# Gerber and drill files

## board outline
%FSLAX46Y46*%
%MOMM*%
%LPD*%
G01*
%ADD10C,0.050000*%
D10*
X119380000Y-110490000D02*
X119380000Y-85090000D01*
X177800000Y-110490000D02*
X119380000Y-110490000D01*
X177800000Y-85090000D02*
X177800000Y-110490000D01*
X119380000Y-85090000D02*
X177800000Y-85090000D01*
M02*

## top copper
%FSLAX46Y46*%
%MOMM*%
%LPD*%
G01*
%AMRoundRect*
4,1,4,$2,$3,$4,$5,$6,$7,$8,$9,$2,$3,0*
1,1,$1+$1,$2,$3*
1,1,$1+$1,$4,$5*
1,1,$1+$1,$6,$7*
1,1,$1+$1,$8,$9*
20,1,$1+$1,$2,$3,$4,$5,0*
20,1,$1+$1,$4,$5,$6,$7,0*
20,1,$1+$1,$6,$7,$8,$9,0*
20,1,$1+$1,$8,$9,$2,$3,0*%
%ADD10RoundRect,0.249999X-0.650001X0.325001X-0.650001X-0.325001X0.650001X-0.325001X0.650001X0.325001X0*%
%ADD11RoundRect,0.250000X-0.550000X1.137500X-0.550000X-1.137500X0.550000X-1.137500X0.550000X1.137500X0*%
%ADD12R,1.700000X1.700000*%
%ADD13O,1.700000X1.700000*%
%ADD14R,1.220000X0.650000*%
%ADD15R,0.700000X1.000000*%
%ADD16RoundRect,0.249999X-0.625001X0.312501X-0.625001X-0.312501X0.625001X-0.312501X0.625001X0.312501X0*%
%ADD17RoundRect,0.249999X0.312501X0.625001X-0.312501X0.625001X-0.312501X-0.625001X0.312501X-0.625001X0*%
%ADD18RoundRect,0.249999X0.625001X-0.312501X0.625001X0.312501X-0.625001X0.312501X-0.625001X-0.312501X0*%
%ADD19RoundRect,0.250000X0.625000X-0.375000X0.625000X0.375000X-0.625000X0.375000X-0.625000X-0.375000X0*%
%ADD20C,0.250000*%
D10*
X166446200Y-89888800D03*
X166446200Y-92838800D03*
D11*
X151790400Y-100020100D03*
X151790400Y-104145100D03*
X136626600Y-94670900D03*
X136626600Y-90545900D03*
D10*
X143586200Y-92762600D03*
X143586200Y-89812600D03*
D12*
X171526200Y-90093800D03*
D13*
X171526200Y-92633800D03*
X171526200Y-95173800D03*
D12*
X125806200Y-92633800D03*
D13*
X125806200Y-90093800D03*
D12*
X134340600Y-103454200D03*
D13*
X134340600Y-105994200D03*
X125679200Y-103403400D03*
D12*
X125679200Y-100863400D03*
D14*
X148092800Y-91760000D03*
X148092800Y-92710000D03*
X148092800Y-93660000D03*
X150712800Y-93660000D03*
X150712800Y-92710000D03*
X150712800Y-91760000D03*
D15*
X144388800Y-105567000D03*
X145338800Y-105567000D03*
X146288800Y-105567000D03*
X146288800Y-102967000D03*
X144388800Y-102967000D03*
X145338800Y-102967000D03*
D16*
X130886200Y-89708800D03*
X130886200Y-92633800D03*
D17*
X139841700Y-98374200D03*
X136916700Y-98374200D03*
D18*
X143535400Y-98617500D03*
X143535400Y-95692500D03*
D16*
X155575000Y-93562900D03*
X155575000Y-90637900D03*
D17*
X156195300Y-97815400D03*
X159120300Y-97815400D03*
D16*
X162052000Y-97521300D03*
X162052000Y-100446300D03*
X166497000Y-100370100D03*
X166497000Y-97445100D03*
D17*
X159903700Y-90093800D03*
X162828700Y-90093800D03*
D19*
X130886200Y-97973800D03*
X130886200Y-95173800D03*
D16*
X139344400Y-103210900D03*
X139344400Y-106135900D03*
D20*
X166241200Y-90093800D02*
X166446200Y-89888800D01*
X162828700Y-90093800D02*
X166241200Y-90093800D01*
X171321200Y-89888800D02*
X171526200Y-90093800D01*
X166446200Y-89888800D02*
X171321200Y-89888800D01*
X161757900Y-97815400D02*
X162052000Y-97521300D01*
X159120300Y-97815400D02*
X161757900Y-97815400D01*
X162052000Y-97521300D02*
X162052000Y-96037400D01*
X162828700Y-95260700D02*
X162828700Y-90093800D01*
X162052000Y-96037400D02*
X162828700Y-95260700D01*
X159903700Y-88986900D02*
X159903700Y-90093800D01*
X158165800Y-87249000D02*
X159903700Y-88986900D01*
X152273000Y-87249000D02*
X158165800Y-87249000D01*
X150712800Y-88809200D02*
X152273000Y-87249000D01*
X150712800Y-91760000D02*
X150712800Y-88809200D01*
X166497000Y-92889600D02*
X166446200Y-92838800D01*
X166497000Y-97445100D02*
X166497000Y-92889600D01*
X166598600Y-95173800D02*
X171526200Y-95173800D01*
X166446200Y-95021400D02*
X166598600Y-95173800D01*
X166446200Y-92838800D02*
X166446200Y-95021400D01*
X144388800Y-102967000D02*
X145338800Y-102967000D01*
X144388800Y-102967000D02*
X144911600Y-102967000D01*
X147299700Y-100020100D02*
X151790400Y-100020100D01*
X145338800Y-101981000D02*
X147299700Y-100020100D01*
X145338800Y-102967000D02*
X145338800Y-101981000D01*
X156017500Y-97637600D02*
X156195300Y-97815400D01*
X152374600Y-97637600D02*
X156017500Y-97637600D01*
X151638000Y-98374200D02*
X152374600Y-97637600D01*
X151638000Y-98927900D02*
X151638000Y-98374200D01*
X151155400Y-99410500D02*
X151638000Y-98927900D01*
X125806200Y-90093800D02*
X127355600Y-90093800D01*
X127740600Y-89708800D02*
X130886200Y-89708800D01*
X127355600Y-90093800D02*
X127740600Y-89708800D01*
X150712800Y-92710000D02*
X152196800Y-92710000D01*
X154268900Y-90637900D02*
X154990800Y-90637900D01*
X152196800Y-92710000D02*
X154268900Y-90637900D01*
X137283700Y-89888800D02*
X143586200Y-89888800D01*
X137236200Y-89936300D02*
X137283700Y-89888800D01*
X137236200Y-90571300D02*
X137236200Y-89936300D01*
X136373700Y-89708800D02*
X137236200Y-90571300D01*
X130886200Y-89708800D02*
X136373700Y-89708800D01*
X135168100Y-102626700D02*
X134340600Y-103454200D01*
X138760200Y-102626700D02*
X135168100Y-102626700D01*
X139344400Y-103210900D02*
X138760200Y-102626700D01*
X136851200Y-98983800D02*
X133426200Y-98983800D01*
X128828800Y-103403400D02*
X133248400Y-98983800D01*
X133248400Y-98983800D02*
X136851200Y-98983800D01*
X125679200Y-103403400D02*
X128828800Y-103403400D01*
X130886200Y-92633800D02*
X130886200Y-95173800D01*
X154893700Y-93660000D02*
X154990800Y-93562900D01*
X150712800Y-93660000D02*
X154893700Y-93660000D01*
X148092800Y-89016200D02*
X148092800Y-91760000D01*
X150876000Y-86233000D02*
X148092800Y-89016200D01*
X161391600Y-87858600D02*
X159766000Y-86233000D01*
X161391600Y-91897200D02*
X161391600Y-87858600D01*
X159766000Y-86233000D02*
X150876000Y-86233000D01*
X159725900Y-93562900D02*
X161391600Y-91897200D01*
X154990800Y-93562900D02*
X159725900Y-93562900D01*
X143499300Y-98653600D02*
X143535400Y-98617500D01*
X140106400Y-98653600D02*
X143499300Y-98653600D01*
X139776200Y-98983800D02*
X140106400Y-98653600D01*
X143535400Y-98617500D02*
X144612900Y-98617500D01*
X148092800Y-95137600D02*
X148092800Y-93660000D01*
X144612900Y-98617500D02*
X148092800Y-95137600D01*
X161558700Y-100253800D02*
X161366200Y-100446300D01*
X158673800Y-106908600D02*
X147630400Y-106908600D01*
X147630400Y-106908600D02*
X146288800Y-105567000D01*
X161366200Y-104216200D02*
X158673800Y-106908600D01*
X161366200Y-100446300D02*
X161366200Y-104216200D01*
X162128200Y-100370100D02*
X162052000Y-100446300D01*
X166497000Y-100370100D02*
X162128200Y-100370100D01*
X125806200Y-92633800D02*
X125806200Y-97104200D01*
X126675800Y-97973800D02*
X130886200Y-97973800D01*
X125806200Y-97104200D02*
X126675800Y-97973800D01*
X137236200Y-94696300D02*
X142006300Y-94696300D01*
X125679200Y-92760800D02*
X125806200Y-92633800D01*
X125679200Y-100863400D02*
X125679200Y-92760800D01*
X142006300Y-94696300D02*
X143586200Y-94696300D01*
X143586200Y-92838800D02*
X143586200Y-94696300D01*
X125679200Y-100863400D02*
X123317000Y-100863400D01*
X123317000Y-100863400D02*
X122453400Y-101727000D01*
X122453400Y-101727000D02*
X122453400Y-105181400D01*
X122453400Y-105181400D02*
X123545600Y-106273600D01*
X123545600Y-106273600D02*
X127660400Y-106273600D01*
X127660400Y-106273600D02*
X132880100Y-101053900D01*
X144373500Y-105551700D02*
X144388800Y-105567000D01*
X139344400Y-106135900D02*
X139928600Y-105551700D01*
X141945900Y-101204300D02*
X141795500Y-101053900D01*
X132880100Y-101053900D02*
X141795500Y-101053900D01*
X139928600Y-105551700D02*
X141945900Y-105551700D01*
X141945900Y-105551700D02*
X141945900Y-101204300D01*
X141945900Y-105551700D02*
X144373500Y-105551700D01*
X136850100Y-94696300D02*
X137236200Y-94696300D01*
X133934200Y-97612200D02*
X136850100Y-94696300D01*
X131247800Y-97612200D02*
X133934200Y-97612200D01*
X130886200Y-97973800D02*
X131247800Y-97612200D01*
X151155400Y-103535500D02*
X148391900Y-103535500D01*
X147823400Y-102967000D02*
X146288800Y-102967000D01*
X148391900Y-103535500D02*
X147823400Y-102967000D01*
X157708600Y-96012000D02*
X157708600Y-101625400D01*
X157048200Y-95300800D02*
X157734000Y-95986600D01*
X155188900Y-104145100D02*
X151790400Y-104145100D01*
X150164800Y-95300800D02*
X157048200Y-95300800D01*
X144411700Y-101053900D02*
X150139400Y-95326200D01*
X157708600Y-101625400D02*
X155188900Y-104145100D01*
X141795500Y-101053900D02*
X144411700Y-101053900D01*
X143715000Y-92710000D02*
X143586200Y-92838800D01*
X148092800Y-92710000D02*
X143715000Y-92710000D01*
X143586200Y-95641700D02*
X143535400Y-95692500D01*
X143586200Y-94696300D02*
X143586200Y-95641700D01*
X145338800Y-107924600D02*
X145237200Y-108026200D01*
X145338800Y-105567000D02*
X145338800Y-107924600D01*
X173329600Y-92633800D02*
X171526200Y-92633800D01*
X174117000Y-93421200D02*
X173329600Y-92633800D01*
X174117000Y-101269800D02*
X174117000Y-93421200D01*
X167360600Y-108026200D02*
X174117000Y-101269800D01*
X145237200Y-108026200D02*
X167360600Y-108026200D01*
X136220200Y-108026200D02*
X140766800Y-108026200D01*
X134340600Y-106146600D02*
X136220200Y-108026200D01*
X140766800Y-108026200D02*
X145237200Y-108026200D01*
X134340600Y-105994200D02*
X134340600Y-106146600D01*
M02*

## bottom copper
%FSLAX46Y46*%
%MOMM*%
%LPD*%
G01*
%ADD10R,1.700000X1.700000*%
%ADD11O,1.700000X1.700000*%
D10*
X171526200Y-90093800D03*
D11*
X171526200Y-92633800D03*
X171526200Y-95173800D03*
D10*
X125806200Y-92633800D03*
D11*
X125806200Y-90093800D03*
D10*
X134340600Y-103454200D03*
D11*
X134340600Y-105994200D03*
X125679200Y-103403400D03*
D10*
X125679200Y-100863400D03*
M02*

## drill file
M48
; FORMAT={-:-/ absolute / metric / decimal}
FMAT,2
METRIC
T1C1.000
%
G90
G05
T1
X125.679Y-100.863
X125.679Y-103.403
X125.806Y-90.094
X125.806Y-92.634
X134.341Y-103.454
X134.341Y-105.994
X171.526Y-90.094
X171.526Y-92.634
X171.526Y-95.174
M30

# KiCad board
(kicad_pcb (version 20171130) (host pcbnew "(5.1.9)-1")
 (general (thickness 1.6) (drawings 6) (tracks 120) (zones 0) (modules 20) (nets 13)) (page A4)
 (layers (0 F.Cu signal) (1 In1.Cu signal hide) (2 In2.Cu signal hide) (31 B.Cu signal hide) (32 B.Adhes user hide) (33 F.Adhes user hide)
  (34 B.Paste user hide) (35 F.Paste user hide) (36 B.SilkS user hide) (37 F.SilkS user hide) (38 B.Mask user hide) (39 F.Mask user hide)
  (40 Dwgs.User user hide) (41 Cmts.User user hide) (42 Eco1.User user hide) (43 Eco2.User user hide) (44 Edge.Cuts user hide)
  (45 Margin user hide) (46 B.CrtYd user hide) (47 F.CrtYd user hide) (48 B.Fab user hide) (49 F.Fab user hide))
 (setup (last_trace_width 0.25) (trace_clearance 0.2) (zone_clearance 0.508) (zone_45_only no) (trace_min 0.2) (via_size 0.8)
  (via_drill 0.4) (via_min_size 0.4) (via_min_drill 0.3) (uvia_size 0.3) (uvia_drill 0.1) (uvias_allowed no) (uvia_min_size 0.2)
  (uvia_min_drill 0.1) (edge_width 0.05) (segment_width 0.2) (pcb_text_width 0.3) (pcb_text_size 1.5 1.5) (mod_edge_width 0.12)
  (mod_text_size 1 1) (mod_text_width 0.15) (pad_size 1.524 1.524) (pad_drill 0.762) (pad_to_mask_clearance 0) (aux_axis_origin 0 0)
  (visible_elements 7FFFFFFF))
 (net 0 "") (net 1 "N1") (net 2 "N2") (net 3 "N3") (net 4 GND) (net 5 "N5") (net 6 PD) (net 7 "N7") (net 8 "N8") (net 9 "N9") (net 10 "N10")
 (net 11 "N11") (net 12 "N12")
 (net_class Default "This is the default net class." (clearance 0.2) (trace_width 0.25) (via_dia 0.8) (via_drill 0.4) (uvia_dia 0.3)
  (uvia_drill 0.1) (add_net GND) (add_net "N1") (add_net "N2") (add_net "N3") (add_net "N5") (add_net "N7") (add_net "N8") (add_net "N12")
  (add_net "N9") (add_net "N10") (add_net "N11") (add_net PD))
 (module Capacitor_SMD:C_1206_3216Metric (layer F.Cu) (at 166.4462 91.3638 270)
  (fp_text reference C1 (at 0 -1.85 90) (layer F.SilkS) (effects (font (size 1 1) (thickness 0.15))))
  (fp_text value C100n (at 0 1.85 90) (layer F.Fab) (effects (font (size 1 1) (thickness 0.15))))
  (pad 1 smd roundrect (at -1.475 0 270) (size 1.15 1.8) (layers F.Cu F.Paste F.Mask) (roundrect_rratio 0.2173904347826087) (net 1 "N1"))
  (pad 2 smd roundrect (at 1.475 0 270) (size 1.15 1.8) (layers F.Cu F.Paste F.Mask) (roundrect_rratio 0.2173904347826087) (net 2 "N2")))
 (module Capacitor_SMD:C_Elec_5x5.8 (layer F.Cu) (at 151.7904 102.0826 270)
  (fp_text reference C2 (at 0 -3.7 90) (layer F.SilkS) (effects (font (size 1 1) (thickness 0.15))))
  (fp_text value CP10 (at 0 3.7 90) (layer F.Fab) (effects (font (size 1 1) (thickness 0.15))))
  (pad 1 smd roundrect (at -2.0625 0 270) (size 2.775 1.6) (layers F.Cu F.Paste F.Mask) (roundrect_rratio 0.15625) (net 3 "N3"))
  (pad 2 smd roundrect (at 2.0625 0 270) (size 2.775 1.6) (layers F.Cu F.Paste F.Mask) (roundrect_rratio 0.15625) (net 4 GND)))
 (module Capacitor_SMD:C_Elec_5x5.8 (layer F.Cu) (at 136.6266 92.6084 270)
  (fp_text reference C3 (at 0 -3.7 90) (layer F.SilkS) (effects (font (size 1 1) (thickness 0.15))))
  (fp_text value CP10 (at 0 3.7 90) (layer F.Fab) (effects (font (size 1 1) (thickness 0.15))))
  (pad 2 smd roundrect (at 2.0625 0 270) (size 2.775 1.6) (layers F.Cu F.Paste F.Mask) (roundrect_rratio 0.15625) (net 4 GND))
  (pad 1 smd roundrect (at -2.0625 0 270) (size 2.775 1.6) (layers F.Cu F.Paste F.Mask) (roundrect_rratio 0.15625) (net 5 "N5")))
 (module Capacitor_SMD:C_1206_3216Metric (layer F.Cu) (at 143.5862 91.2876 270)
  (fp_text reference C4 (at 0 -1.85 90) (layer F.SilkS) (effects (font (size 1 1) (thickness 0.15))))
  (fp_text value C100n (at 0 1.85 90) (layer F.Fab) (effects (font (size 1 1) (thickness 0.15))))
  (pad 2 smd roundrect (at 1.475 0 270) (size 1.15 1.8) (layers F.Cu F.Paste F.Mask) (roundrect_rratio 0.2173904347826087) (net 4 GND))
  (pad 1 smd roundrect (at -1.475 0 270) (size 1.15 1.8) (layers F.Cu F.Paste F.Mask) (roundrect_rratio 0.2173904347826087) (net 5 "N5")))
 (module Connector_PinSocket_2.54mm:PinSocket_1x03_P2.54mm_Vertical (layer F.Cu) (at 171.5262 90.0938)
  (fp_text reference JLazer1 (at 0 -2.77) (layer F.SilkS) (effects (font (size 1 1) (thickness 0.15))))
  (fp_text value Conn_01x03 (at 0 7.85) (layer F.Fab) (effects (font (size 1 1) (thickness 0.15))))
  (pad 1 thru_hole rect (at 0 0) (size 1.7 1.7) (drill 1) (layers *.Cu *.Mask) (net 1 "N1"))
  (pad 2 thru_hole oval (at 0 2.54) (size 1.7 1.7) (drill 1) (layers *.Cu *.Mask) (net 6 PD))
  (pad 3 thru_hole oval (at 0 5.08) (size 1.7 1.7) (drill 1) (layers *.Cu *.Mask) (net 2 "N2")))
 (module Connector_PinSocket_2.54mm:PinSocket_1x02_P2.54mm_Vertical (layer F.Cu) (at 125.8062 92.6338 180)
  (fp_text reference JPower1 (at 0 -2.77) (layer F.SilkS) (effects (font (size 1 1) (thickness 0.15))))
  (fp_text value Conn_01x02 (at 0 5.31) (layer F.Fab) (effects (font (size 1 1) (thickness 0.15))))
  (pad 1 thru_hole rect (at 0 0 180) (size 1.7 1.7) (drill 1) (layers *.Cu *.Mask) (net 4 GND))
  (pad 2 thru_hole oval (at 0 2.54 180) (size 1.7 1.7) (drill 1) (layers *.Cu *.Mask) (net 5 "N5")))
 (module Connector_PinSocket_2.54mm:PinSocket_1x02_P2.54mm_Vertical (layer F.Cu) (at 134.3406 103.4542)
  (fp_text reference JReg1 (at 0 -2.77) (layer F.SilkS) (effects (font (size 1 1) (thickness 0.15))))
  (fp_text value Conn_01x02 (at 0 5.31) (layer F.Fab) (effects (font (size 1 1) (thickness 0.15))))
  (pad 1 thru_hole rect (at 0 0) (size 1.7 1.7) (drill 1) (layers *.Cu *.Mask) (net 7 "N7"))
  (pad 2 thru_hole oval (at 0 2.54) (size 1.7 1.7) (drill 1) (layers *.Cu *.Mask) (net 6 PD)))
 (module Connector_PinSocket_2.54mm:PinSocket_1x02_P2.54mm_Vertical (layer F.Cu) (at 125.6792 100.8634)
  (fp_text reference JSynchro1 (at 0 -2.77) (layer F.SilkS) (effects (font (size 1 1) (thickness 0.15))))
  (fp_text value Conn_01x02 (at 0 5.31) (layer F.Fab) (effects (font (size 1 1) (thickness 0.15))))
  (pad 2 thru_hole oval (at 0 2.54) (size 1.7 1.7) (drill 1) (layers *.Cu *.Mask) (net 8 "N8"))
  (pad 1 thru_hole rect (at 0 0) (size 1.7 1.7) (drill 1) (layers *.Cu *.Mask) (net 4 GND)))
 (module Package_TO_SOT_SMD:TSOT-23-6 (layer F.Cu) (at 149.4028 92.71)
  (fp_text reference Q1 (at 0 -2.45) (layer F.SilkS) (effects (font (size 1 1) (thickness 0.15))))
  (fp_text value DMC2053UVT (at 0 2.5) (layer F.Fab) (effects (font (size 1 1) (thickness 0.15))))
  (pad 1 smd rect (at -1.31 -0.95) (size 1.22 0.65) (layers F.Cu F.Paste F.Mask) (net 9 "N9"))
  (pad 2 smd rect (at -1.31 0) (size 1.22 0.65) (layers F.Cu F.Paste F.Mask) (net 4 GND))
  (pad 3 smd rect (at -1.31 0.95) (size 1.22 0.65) (layers F.Cu F.Paste F.Mask) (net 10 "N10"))
  (pad 4 smd rect (at 1.31 0.95) (size 1.22 0.65) (layers F.Cu F.Paste F.Mask) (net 9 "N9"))
  (pad 5 smd rect (at 1.31 0) (size 1.22 0.65) (layers F.Cu F.Paste F.Mask) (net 5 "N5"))
  (pad 6 smd rect (at 1.31 -0.95) (size 1.22 0.65) (layers F.Cu F.Paste F.Mask) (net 1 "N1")))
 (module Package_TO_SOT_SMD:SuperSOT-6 (layer F.Cu) (at 145.3388 104.267 90)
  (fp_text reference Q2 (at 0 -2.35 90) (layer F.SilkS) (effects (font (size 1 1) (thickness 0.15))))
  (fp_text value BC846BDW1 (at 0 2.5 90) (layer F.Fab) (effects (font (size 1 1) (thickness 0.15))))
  (pad 1 smd rect (at -1.3 -0.95 90) (size 1 0.7) (layers F.Cu F.Paste F.Mask) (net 4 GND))
  (pad 2 smd rect (at -1.3 0 90) (size 1 0.7) (layers F.Cu F.Paste F.Mask) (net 6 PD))
  (pad 3 smd rect (at -1.3 0.95 90) (size 1 0.7) (layers F.Cu F.Paste F.Mask) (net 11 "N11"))
  (pad 4 smd rect (at 1.3 0.95 90) (size 1 0.7) (layers F.Cu F.Paste F.Mask) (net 4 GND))
  (pad 6 smd rect (at 1.3 -0.95 90) (size 1 0.7) (layers F.Cu F.Paste F.Mask) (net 3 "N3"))
  (pad 5 smd rect (at 1.3 0 90) (size 1 0.7) (layers F.Cu F.Paste F.Mask) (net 3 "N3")))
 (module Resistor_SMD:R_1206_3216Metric (layer F.Cu) (at 130.8862 91.1713 270)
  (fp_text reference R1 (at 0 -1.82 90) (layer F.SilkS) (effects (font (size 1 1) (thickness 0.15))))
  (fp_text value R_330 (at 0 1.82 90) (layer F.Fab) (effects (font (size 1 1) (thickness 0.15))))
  (pad 1 smd roundrect (at -1.4625 0 270) (size 1.125 1.75) (layers F.Cu F.Paste F.Mask) (roundrect_rratio 0.2222213333333333) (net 5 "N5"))
  (pad 2 smd roundrect (at 1.4625 0 270) (size 1.125 1.75) (layers F.Cu F.Paste F.Mask) (roundrect_rratio 0.2222213333333333) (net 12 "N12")))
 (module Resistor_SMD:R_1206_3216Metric (layer F.Cu) (at 138.3792 98.3742 180)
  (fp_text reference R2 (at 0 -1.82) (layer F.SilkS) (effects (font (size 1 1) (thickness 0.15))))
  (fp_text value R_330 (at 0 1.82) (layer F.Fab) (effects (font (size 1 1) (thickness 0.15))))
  (pad 1 smd roundrect (at -1.4625 0 180) (size 1.125 1.75) (layers F.Cu F.Paste F.Mask) (roundrect_rratio 0.2222213333333333)
   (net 10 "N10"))
  (pad 2 smd roundrect (at 1.4625 0 180) (size 1.125 1.75) (layers F.Cu F.Paste F.Mask) (roundrect_rratio 0.2222213333333333) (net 8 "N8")))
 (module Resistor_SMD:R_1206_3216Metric (layer F.Cu) (at 143.5354 97.155 90)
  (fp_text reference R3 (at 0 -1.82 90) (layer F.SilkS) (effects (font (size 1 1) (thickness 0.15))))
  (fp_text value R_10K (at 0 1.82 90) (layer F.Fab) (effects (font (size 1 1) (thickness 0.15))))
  (pad 1 smd roundrect (at -1.4625 0 90) (size 1.125 1.75) (layers F.Cu F.Paste F.Mask) (roundrect_rratio 0.2222213333333333) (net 10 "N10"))
  (pad 2 smd roundrect (at 1.4625 0 90) (size 1.125 1.75) (layers F.Cu F.Paste F.Mask) (roundrect_rratio 0.2222213333333333) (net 4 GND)))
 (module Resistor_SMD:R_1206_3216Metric (layer F.Cu) (at 155.575 92.1004 270)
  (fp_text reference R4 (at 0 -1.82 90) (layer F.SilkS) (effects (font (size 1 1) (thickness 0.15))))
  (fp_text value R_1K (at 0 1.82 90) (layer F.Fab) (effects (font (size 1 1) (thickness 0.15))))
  (pad 2 smd roundrect (at 1.4625 0 270) (size 1.125 1.75) (layers F.Cu F.Paste F.Mask) (roundrect_rratio 0.2222213333333333) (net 9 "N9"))
  (pad 1 smd roundrect (at -1.4625 0 270) (size 1.125 1.75) (layers F.Cu F.Paste F.Mask) (roundrect_rratio 0.2222213333333333) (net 5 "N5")))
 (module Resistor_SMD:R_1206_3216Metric (layer F.Cu) (at 157.6578 97.8154 180)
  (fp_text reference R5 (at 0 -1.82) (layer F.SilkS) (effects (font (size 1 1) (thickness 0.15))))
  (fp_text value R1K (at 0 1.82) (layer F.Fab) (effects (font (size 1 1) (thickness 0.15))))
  (pad 2 smd roundrect (at 1.4625 0 180) (size 1.125 1.75) (layers F.Cu F.Paste F.Mask) (roundrect_rratio 0.2222213333333333) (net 3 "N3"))
  (pad 1 smd roundrect (at -1.4625 0 180) (size 1.125 1.75) (layers F.Cu F.Paste F.Mask) (roundrect_rratio 0.2222213333333333) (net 1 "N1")))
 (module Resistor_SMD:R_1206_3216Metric (layer F.Cu) (at 162.052 98.9838 270)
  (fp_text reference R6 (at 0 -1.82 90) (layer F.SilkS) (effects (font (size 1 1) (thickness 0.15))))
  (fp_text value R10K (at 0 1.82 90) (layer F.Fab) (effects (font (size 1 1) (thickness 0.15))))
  (pad 1 smd roundrect (at -1.4625 0 270) (size 1.125 1.75) (layers F.Cu F.Paste F.Mask) (roundrect_rratio 0.2222213333333333) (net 1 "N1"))
  (pad 2 smd roundrect (at 1.4625 0 270) (size 1.125 1.75) (layers F.Cu F.Paste F.Mask) (roundrect_rratio 0.2222213333333333) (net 11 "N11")))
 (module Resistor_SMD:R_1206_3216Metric (layer F.Cu) (at 166.497 98.9076 270)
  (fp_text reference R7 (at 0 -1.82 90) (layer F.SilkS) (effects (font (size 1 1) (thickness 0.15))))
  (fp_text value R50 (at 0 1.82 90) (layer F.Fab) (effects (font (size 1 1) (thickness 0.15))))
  (pad 2 smd roundrect (at 1.4625 0 270) (size 1.125 1.75) (layers F.Cu F.Paste F.Mask) (roundrect_rratio 0.2222213333333333) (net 11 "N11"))
  (pad 1 smd roundrect (at -1.4625 0 270) (size 1.125 1.75) (layers F.Cu F.Paste F.Mask) (roundrect_rratio 0.2222213333333333) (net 2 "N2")))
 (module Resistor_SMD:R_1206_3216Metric (layer F.Cu) (at 161.3662 90.0938 180)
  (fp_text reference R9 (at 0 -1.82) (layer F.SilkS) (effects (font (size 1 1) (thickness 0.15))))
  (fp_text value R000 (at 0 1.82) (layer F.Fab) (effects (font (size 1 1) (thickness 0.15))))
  (pad 2 smd roundrect (at 1.4625 0 180) (size 1.125 1.75) (layers F.Cu F.Paste F.Mask) (roundrect_rratio 0.2222213333333333) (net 1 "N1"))
  (pad 1 smd roundrect (at -1.4625 0 180) (size 1.125 1.75) (layers F.Cu F.Paste F.Mask) (roundrect_rratio 0.2222213333333333) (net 1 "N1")))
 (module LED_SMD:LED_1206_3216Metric (layer F.Cu) (at 130.8862 96.5738 90)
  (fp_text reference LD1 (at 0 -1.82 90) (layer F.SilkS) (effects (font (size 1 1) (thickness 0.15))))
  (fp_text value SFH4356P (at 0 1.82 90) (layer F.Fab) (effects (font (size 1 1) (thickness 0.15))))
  (pad 1 smd roundrect (at -1.4 0 90) (size 1.25 1.75) (layers F.Cu F.Paste F.Mask) (roundrect_rratio 0.2) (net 4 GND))
  (pad 2 smd roundrect (at 1.4 0 90) (size 1.25 1.75) (layers F.Cu F.Paste F.Mask) (roundrect_rratio 0.2) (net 12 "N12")))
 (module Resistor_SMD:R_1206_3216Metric (layer F.Cu) (at 139.3444 104.6734 270)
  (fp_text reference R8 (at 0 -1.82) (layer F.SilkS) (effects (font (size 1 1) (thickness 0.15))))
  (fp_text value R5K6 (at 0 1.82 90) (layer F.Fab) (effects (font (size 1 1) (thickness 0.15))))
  (pad 1 smd roundrect (at -1.4625 0 270) (size 1.125 1.75) (layers F.Cu F.Paste F.Mask) (roundrect_rratio 0.2222213333333333) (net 7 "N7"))
  (pad 2 smd roundrect (at 1.4625 0 270) (size 1.125 1.75) (layers F.Cu F.Paste F.Mask) (roundrect_rratio 0.2222213333333333) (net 4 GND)))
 (gr_line (start 119.38 110.49) (end 119.38 85.09) (layer Edge.Cuts) (width 0.05))
 (gr_line (start 177.8 110.49) (end 119.38 110.49) (layer Edge.Cuts) (width 0.05))
 (gr_line (start 177.8 85.09) (end 177.8 110.49) (layer Edge.Cuts) (width 0.05))
 (gr_line (start 119.38 85.09) (end 177.8 85.09) (layer Edge.Cuts) (width 0.05))
 (segment (start 166.2412 90.0938) (end 166.4462 89.8888) (width 0.25) (layer F.Cu) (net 1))
 (segment (start 162.8287 90.0938) (end 166.2412 90.0938) (width 0.25) (layer F.Cu) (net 1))
 (segment (start 171.3212 89.8888) (end 171.5262 90.0938) (width 0.25) (layer F.Cu) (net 1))
 (segment (start 166.4462 89.8888) (end 171.3212 89.8888) (width 0.25) (layer F.Cu) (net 1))
 (segment (start 161.7579 97.8154) (end 162.052 97.5213) (width 0.25) (layer F.Cu) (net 1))
 (segment (start 159.1203 97.8154) (end 161.7579 97.8154) (width 0.25) (layer F.Cu) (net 1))
 (segment (start 162.052 97.5213) (end 162.052 96.0374) (width 0.25) (layer F.Cu) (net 1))
 (segment (start 162.8287 95.2607) (end 162.8287 90.0938) (width 0.25) (layer F.Cu) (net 1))
 (segment (start 162.052 96.0374) (end 162.8287 95.2607) (width 0.25) (layer F.Cu) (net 1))
 (segment (start 159.9037 88.9869) (end 159.9037 90.0938) (width 0.25) (layer F.Cu) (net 1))
 (segment (start 158.1658 87.249) (end 159.9037 88.9869) (width 0.25) (layer F.Cu) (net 1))
 (segment (start 152.273 87.249) (end 158.1658 87.249) (width 0.25) (layer F.Cu) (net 1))
 (segment (start 150.7128 88.8092) (end 152.273 87.249) (width 0.25) (layer F.Cu) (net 1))
 (segment (start 150.7128 91.76) (end 150.7128 88.8092) (width 0.25) (layer F.Cu) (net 1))
 (segment (start 166.497 92.8896) (end 166.4462 92.8388) (width 0.25) (layer F.Cu) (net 2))
 (segment (start 166.497 97.4451) (end 166.497 92.8896) (width 0.25) (layer F.Cu) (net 2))
 (segment (start 166.5986 95.1738) (end 171.5262 95.1738) (width 0.25) (layer F.Cu) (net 2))
 (segment (start 166.4462 95.0214) (end 166.5986 95.1738) (width 0.25) (layer F.Cu) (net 2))
 (segment (start 166.4462 92.8388) (end 166.4462 95.0214) (width 0.25) (layer F.Cu) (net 2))
 (segment (start 144.3888 102.967) (end 145.3388 102.967) (width 0.25) (layer F.Cu) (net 3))
 (segment (start 144.3888 102.967) (end 144.9116 102.967) (width 0.25) (layer F.Cu) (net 3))
 (segment (start 147.2997 100.0201) (end 151.7904 100.0201) (width 0.25) (layer F.Cu) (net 3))
 (segment (start 145.3388 101.981) (end 147.2997 100.0201) (width 0.25) (layer F.Cu) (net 3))
 (segment (start 145.3388 102.967) (end 145.3388 101.981) (width 0.25) (layer F.Cu) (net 3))
 (segment (start 156.0175 97.6376) (end 156.1953 97.8154) (width 0.25) (layer F.Cu) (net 3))
 (segment (start 152.3746 97.6376) (end 156.0175 97.6376) (width 0.25) (layer F.Cu) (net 3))
 (segment (start 151.638 98.3742) (end 152.3746 97.6376) (width 0.25) (layer F.Cu) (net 3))
 (segment (start 151.638 98.9279) (end 151.638 98.3742) (width 0.25) (layer F.Cu) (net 3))
 (segment (start 151.1554 99.4105) (end 151.638 98.9279) (width 0.25) (layer F.Cu) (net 3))
 (segment (start 125.8062 90.0938) (end 127.3556 90.0938) (width 0.25) (layer F.Cu) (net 5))
 (segment (start 127.7406 89.7088) (end 130.8862 89.7088) (width 0.25) (layer F.Cu) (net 5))
 (segment (start 127.3556 90.0938) (end 127.7406 89.7088) (width 0.25) (layer F.Cu) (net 5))
 (segment (start 150.7128 92.71) (end 152.1968 92.71) (width 0.25) (layer F.Cu) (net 5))
 (segment (start 154.2689 90.6379) (end 154.9908 90.6379) (width 0.25) (layer F.Cu) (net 5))
 (segment (start 152.1968 92.71) (end 154.2689 90.6379) (width 0.25) (layer F.Cu) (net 5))
 (segment (start 137.2837 89.8888) (end 143.5862 89.8888) (width 0.25) (layer F.Cu) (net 5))
 (segment (start 137.2362 89.9363) (end 137.2837 89.8888) (width 0.25) (layer F.Cu) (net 5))
 (segment (start 137.2362 90.5713) (end 137.2362 89.9363) (width 0.25) (layer F.Cu) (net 5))
 (segment (start 136.3737 89.7088) (end 137.2362 90.5713) (width 0.25) (layer F.Cu) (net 5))
 (segment (start 130.8862 89.7088) (end 136.3737 89.7088) (width 0.25) (layer F.Cu) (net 5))
 (segment (start 135.1681 102.6267) (end 134.3406 103.4542) (width 0.25) (layer F.Cu) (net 7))
 (segment (start 138.7602 102.6267) (end 135.1681 102.6267) (width 0.25) (layer F.Cu) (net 7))
 (segment (start 139.3444 103.2109) (end 138.7602 102.6267) (width 0.25) (layer F.Cu) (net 7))
 (segment (start 136.8512 98.9838) (end 133.4262 98.9838) (width 0.25) (layer F.Cu) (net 8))
 (segment (start 128.8288 103.4034) (end 133.2484 98.9838) (width 0.25) (layer F.Cu) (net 8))
 (segment (start 133.2484 98.9838) (end 136.8512 98.9838) (width 0.25) (layer F.Cu) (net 8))
 (segment (start 125.6792 103.4034) (end 128.8288 103.4034) (width 0.25) (layer F.Cu) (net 8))
 (segment (start 130.8862 92.6338) (end 130.8862 95.1738) (width 0.25) (layer F.Cu) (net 12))
 (segment (start 154.8937 93.66) (end 154.9908 93.5629) (width 0.25) (layer F.Cu) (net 9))
 (segment (start 150.7128 93.66) (end 154.8937 93.66) (width 0.25) (layer F.Cu) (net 9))
 (segment (start 148.0928 89.0162) (end 148.0928 91.76) (width 0.25) (layer F.Cu) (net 9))
 (segment (start 150.876 86.233) (end 148.0928 89.0162) (width 0.25) (layer F.Cu) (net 9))
 (segment (start 161.3916 87.8586) (end 159.766 86.233) (width 0.25) (layer F.Cu) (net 9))
 (segment (start 161.3916 91.8972) (end 161.3916 87.8586) (width 0.25) (layer F.Cu) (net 9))
 (segment (start 159.766 86.233) (end 150.876 86.233) (width 0.25) (layer F.Cu) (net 9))
 (segment (start 159.7259 93.5629) (end 161.3916 91.8972) (width 0.25) (layer F.Cu) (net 9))
 (segment (start 154.9908 93.5629) (end 159.7259 93.5629) (width 0.25) (layer F.Cu) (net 9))
 (segment (start 143.4993 98.6536) (end 143.5354 98.6175) (width 0.25) (layer F.Cu) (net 10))
 (segment (start 140.1064 98.6536) (end 143.4993 98.6536) (width 0.25) (layer F.Cu) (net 10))
 (segment (start 139.7762 98.9838) (end 140.1064 98.6536) (width 0.25) (layer F.Cu) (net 10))
 (segment (start 143.5354 98.6175) (end 144.6129 98.6175) (width 0.25) (layer F.Cu) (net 10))
 (segment (start 148.0928 95.1376) (end 148.0928 93.66) (width 0.25) (layer F.Cu) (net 10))
 (segment (start 144.6129 98.6175) (end 148.0928 95.1376) (width 0.25) (layer F.Cu) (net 10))
 (segment (start 161.5587 100.2538) (end 161.3662 100.4463) (width 0.25) (layer F.Cu) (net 11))
 (segment (start 158.6738 106.9086) (end 147.6304 106.9086) (width 0.25) (layer F.Cu) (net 11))
 (segment (start 147.6304 106.9086) (end 146.2888 105.567) (width 0.25) (layer F.Cu) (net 11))
 (segment (start 161.3662 104.2162) (end 158.6738 106.9086) (width 0.25) (layer F.Cu) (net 11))
 (segment (start 161.3662 100.4463) (end 161.3662 104.2162) (width 0.25) (layer F.Cu) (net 11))
 (segment (start 162.1282 100.3701) (end 162.052 100.4463) (width 0.25) (layer F.Cu) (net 11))
 (segment (start 166.497 100.3701) (end 162.1282 100.3701) (width 0.25) (layer F.Cu) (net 11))
 (segment (start 125.8062 92.6338) (end 125.8062 97.1042) (width 0.25) (layer F.Cu) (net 4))
 (segment (start 126.6758 97.9738) (end 130.8862 97.9738) (width 0.25) (layer F.Cu) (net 4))
 (segment (start 125.8062 97.1042) (end 126.6758 97.9738) (width 0.25) (layer F.Cu) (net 4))
 (segment (start 137.2362 94.6963) (end 142.0063 94.6963) (width 0.25) (layer F.Cu) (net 4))
 (segment (start 125.6792 92.7608) (end 125.8062 92.6338) (width 0.25) (layer F.Cu) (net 4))
 (segment (start 125.6792 100.8634) (end 125.6792 92.7608) (width 0.25) (layer F.Cu) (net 4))
 (segment (start 142.0063 94.6963) (end 143.5862 94.6963) (width 0.25) (layer F.Cu) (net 4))
 (segment (start 143.5862 92.8388) (end 143.5862 94.6963) (width 0.25) (layer F.Cu) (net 4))
 (segment (start 125.6792 100.8634) (end 123.317 100.8634) (width 0.25) (layer F.Cu) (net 4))
 (segment (start 123.317 100.8634) (end 122.4534 101.727) (width 0.25) (layer F.Cu) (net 4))
 (segment (start 122.4534 101.727) (end 122.4534 105.1814) (width 0.25) (layer F.Cu) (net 4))
 (segment (start 122.4534 105.1814) (end 123.5456 106.2736) (width 0.25) (layer F.Cu) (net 4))
 (segment (start 123.5456 106.2736) (end 127.6604 106.2736) (width 0.25) (layer F.Cu) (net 4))
 (segment (start 127.6604 106.2736) (end 132.8801 101.0539) (width 0.25) (layer F.Cu) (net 4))
 (segment (start 144.3735 105.5517) (end 144.3888 105.567) (width 0.25) (layer F.Cu) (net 4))
 (segment (start 139.3444 106.1359) (end 139.9286 105.5517) (width 0.25) (layer F.Cu) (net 4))
 (segment (start 141.9459 101.2043) (end 141.7955 101.0539) (width 0.25) (layer F.Cu) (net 4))
 (segment (start 132.8801 101.0539) (end 141.7955 101.0539) (width 0.25) (layer F.Cu) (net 4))
 (segment (start 139.9286 105.5517) (end 141.9459 105.5517) (width 0.25) (layer F.Cu) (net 4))
 (segment (start 141.9459 105.5517) (end 141.9459 101.2043) (width 0.25) (layer F.Cu) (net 4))
 (segment (start 141.9459 105.5517) (end 144.3735 105.5517) (width 0.25) (layer F.Cu) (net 4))
 (segment (start 136.8501 94.6963) (end 137.2362 94.6963) (width 0.25) (layer F.Cu) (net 4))
 (segment (start 133.9342 97.6122) (end 136.8501 94.6963) (width 0.25) (layer F.Cu) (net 4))
 (segment (start 131.2478 97.6122) (end 133.9342 97.6122) (width 0.25) (layer F.Cu) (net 4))
 (segment (start 130.8862 97.9738) (end 131.2478 97.6122) (width 0.25) (layer F.Cu) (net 4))
 (segment (start 151.1554 103.5355) (end 148.3919 103.5355) (width 0.25) (layer F.Cu) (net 4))
 (segment (start 147.8234 102.967) (end 146.2888 102.967) (width 0.25) (layer F.Cu) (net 4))
 (segment (start 148.3919 103.5355) (end 147.8234 102.967) (width 0.25) (layer F.Cu) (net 4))
 (segment (start 157.7086 96.012) (end 157.7086 101.6254) (width 0.25) (layer F.Cu) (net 4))
 (segment (start 157.0482 95.3008) (end 157.734 95.9866) (width 0.25) (layer F.Cu) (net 4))
 (segment (start 155.1889 104.1451) (end 151.7904 104.1451) (width 0.25) (layer F.Cu) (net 4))
 (segment (start 150.1648 95.3008) (end 157.0482 95.3008) (width 0.25) (layer F.Cu) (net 4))
 (segment (start 144.4117 101.0539) (end 150.1394 95.3262) (width 0.25) (layer F.Cu) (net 4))
 (segment (start 157.7086 101.6254) (end 155.1889 104.1451) (width 0.25) (layer F.Cu) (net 4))
 (segment (start 141.7955 101.0539) (end 144.4117 101.0539) (width 0.25) (layer F.Cu) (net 4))
 (segment (start 143.715 92.71) (end 143.5862 92.8388) (width 0.25) (layer F.Cu) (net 4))
 (segment (start 148.0928 92.71) (end 143.715 92.71) (width 0.25) (layer F.Cu) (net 4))
 (segment (start 143.5862 95.6417) (end 143.5354 95.6925) (width 0.25) (layer F.Cu) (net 4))
 (segment (start 143.5862 94.6963) (end 143.5862 95.6417) (width 0.25) (layer F.Cu) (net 4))
 (segment (start 145.3388 107.9246) (end 145.2372 108.0262) (width 0.25) (layer F.Cu) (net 6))
 (segment (start 145.3388 105.567) (end 145.3388 107.9246) (width 0.25) (layer F.Cu) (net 6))
 (segment (start 173.3296 92.6338) (end 171.5262 92.6338) (width 0.25) (layer F.Cu) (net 6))
 (segment (start 174.117 93.4212) (end 173.3296 92.6338) (width 0.25) (layer F.Cu) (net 6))
 (segment (start 174.117 101.2698) (end 174.117 93.4212) (width 0.25) (layer F.Cu) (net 6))
 (segment (start 167.3606 108.0262) (end 174.117 101.2698) (width 0.25) (layer F.Cu) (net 6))
 (segment (start 145.2372 108.0262) (end 167.3606 108.0262) (width 0.25) (layer F.Cu) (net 6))
 (segment (start 136.2202 108.0262) (end 140.7668 108.0262) (width 0.25) (layer F.Cu) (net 6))
 (segment (start 134.3406 106.1466) (end 136.2202 108.0262) (width 0.25) (layer F.Cu) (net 6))
 (segment (start 140.7668 108.0262) (end 145.2372 108.0262) (width 0.25) (layer F.Cu) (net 6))
 (segment (start 134.3406 105.9942) (end 134.3406 106.1466) (width 0.25) (layer F.Cu) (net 6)))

